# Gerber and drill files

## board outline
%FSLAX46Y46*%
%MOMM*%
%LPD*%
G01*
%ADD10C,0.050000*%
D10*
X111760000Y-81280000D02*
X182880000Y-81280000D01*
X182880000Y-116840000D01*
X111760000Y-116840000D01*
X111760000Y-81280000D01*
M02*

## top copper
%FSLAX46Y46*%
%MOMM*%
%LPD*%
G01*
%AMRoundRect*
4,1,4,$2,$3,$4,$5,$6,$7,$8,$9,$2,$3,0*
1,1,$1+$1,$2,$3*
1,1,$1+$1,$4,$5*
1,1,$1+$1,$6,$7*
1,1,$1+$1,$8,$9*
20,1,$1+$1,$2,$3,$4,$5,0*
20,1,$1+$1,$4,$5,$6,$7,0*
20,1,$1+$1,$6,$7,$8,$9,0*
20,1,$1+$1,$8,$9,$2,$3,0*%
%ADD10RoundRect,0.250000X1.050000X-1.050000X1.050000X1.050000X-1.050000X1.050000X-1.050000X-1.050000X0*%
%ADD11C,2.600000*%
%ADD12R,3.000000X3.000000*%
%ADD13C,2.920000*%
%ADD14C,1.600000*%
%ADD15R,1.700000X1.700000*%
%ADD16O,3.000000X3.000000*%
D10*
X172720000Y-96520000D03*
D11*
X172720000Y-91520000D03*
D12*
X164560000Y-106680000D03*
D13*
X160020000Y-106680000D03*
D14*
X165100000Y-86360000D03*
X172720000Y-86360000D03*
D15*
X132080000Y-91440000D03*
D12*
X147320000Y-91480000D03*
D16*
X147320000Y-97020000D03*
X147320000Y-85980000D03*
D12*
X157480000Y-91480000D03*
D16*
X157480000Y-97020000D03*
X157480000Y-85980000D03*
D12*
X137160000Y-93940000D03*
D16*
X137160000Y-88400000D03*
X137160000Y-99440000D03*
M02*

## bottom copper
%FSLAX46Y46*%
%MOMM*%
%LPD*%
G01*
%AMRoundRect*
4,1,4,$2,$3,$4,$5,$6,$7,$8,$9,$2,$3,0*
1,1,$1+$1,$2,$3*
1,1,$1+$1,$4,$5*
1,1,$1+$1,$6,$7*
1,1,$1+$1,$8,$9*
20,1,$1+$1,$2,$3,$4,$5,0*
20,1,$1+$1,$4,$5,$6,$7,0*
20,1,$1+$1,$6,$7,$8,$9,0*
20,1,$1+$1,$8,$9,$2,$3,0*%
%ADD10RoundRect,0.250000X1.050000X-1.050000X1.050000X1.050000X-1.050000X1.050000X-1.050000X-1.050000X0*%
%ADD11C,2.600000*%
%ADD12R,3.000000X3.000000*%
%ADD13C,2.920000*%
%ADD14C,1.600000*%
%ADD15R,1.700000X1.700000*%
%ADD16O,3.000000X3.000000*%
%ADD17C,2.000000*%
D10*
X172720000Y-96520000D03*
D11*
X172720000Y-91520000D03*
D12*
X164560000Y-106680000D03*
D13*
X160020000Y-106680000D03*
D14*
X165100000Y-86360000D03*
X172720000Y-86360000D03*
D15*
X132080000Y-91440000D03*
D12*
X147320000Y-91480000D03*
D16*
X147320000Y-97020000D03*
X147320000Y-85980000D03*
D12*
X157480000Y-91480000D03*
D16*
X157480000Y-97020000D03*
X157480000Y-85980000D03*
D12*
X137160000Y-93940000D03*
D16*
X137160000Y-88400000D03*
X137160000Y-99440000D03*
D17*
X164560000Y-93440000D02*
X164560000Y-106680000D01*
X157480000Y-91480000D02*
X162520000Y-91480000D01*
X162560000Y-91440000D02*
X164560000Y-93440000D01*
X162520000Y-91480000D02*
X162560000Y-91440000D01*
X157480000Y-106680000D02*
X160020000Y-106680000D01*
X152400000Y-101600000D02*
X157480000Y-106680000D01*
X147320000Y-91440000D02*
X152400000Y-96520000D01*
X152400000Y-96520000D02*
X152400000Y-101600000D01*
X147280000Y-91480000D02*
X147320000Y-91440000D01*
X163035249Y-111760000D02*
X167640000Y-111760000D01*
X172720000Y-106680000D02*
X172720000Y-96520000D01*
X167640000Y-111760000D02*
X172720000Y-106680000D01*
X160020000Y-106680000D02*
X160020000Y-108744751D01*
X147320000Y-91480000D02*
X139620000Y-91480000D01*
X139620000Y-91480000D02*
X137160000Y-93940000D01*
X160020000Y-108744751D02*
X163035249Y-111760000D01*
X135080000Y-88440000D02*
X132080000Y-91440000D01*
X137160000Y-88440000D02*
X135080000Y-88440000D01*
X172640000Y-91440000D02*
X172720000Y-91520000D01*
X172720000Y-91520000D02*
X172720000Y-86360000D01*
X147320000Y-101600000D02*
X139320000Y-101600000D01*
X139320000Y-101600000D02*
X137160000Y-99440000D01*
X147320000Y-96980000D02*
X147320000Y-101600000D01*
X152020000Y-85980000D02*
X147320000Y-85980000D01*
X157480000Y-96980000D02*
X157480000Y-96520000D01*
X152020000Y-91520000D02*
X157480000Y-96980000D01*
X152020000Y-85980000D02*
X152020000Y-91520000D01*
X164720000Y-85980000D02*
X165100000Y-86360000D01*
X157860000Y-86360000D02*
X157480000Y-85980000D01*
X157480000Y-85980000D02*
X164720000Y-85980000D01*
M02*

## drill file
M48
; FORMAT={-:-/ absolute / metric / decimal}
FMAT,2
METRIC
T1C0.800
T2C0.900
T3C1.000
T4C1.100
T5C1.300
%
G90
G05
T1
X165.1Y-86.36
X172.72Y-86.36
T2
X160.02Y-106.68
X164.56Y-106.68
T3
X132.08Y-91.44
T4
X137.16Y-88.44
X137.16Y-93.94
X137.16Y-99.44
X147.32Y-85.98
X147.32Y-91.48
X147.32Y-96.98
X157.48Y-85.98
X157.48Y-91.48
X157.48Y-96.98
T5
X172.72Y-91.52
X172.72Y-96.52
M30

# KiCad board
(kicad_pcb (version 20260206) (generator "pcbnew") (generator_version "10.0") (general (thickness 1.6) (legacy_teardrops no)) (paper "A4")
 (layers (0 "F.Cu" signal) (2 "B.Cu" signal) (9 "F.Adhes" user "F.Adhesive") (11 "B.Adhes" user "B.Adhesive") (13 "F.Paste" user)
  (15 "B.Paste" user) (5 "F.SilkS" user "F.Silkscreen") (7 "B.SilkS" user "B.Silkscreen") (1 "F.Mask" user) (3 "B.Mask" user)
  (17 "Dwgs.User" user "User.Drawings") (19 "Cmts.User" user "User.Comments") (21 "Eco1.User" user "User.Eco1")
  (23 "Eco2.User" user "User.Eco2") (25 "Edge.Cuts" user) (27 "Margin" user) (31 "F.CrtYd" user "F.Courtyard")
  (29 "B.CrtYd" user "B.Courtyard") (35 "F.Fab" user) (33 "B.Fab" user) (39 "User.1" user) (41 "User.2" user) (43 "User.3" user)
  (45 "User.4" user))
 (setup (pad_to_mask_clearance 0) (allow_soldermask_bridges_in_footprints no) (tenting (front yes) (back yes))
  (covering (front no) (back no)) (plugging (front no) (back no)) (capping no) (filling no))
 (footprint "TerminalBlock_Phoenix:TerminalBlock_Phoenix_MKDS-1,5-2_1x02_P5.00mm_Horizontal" (layer "F.Cu") (at 172.72 96.52 90)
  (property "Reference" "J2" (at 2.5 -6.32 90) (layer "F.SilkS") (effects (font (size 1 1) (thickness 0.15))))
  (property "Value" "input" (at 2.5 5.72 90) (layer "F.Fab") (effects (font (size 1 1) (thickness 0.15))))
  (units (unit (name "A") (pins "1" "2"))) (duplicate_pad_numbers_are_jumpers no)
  (pad "1" thru_hole roundrect (at 0 0 90) (size 2.6 2.6) (drill 1.3) (layers "*.Cu" "*.Mask") (remove_unused_layers no)
   (roundrect_rratio 0.096154) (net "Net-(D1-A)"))
  (pad "2" thru_hole circle (at 5 0 90) (size 2.6 2.6) (drill 1.3) (layers "*.Cu" "*.Mask") (remove_unused_layers no) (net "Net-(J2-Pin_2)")))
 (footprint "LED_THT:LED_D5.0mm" (layer "F.Cu") (at 162.56 106.68 180)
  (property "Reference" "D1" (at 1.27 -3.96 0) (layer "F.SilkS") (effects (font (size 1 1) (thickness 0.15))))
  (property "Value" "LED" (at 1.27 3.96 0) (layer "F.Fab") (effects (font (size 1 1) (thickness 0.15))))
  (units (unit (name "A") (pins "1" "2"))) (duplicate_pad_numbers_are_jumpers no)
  (pad "1" thru_hole rect (at -2 0 180) (size 3 3) (drill 0.9) (layers "*.Cu" "*.Mask") (remove_unused_layers no) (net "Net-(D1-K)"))
  (pad "2" thru_hole circle (at 2.54 0 180) (size 2.92 2.92) (drill 0.9) (layers "*.Cu" "*.Mask") (remove_unused_layers no)
   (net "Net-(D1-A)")))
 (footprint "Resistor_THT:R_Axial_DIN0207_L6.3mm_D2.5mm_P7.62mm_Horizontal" (layer "F.Cu") (at 165.1 86.36)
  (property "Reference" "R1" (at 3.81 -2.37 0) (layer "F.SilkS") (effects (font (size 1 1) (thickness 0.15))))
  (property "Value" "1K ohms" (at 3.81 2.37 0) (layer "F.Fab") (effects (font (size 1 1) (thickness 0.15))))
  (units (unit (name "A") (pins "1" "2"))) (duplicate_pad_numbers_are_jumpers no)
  (pad "1" thru_hole circle (at 0 0) (size 1.6 1.6) (drill 0.8) (layers "*.Cu" "*.Mask") (remove_unused_layers no) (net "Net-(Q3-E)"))
  (pad "2" thru_hole circle (at 7.62 0) (size 1.6 1.6) (drill 0.8) (layers "*.Cu" "*.Mask") (remove_unused_layers no) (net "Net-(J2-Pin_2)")))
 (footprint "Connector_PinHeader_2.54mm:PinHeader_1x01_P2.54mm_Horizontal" (layer "F.Cu") (at 132.08 91.44 180)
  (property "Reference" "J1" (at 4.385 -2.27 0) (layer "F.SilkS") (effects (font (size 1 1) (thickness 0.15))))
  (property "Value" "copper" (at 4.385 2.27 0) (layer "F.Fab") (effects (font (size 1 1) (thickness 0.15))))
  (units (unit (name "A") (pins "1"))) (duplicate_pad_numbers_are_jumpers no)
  (pad "1" thru_hole rect (at 0 0 180) (size 1.7 1.7) (drill 1) (layers "*.Cu" "*.Mask") (remove_unused_layers no) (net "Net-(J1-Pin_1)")))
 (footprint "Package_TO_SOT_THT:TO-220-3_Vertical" (layer "F.Cu") (at 147.32 93.98 90)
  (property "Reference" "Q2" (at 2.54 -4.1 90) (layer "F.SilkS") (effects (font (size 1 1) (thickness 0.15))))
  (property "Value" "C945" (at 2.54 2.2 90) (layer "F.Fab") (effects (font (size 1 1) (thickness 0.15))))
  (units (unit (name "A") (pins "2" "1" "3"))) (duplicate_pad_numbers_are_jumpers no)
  (pad "1" thru_hole rect (at 2.5 0 90) (size 3 3) (drill 1.1) (layers "*.Cu" "*.Mask") (remove_unused_layers no) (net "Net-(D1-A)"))
  (pad "2" thru_hole oval (at -3 0 90) (size 3 3) (drill 1.1 (offset -0.04 0)) (layers "*.Cu" "*.Mask") (remove_unused_layers no)
   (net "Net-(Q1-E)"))
  (pad "3" thru_hole oval (at 8 0 90) (size 3 3) (drill 1.1) (layers "*.Cu" "*.Mask") (remove_unused_layers no) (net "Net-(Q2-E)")))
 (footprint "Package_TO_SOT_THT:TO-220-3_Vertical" (layer "F.Cu") (at 157.48 93.98 90)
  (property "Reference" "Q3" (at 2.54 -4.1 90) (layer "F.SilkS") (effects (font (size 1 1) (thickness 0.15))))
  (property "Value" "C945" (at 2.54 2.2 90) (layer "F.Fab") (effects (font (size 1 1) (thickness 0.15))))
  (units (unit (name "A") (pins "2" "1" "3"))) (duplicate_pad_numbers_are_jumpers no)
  (pad "1" thru_hole rect (at 2.5 0 90) (size 3 3) (drill 1.1) (layers "*.Cu" "*.Mask") (remove_unused_layers no) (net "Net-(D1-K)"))
  (pad "2" thru_hole oval (at -3 0 90) (size 3 3) (drill 1.1 (offset -0.04 0)) (layers "*.Cu" "*.Mask") (remove_unused_layers no)
   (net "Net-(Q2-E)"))
  (pad "3" thru_hole oval (at 8 0 90) (size 3 3) (drill 1.1) (layers "*.Cu" "*.Mask") (remove_unused_layers no) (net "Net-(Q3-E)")))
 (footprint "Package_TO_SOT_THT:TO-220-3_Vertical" (layer "F.Cu") (at 137.16 91.44 -90)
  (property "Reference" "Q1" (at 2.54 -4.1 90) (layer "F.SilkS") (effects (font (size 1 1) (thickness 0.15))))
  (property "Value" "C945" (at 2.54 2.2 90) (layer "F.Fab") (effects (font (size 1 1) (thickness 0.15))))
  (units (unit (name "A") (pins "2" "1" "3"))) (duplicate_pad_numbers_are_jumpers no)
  (pad "1" thru_hole rect (at 2.5 0 270) (size 3 3) (drill 1.1) (layers "*.Cu" "*.Mask") (remove_unused_layers no) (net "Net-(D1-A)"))
  (pad "2" thru_hole oval (at -3 0 270) (size 3 3) (drill 1.1 (offset -0.04 0)) (layers "*.Cu" "*.Mask") (remove_unused_layers no)
   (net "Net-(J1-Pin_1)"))
  (pad "3" thru_hole oval (at 8 0 270) (size 3 3) (drill 1.1) (layers "*.Cu" "*.Mask") (remove_unused_layers no) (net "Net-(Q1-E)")))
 (gr_rect (start 111.76 81.28) (end 182.88 116.84) (stroke (width 0.05) (type default)) (fill no) (layer "Edge.Cuts"))
 (segment (start 164.56 93.44) (end 164.56 106.68) (width 2) (layer "B.Cu") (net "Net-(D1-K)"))
 (segment (start 157.48 91.48) (end 162.52 91.48) (width 2) (layer "B.Cu") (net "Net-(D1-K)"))
 (segment (start 162.56 91.44) (end 164.56 93.44) (width 2) (layer "B.Cu") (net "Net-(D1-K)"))
 (segment (start 162.52 91.48) (end 162.56 91.44) (width 2) (layer "B.Cu") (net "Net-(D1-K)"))
 (segment (start 157.48 106.68) (end 160.02 106.68) (width 2) (layer "B.Cu") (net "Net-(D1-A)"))
 (segment (start 152.4 101.6) (end 157.48 106.68) (width 2) (layer "B.Cu") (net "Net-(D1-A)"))
 (segment (start 147.32 91.44) (end 152.4 96.52) (width 2) (layer "B.Cu") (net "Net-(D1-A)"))
 (segment (start 152.4 96.52) (end 152.4 101.6) (width 2) (layer "B.Cu") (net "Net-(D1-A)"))
 (segment (start 147.28 91.48) (end 147.32 91.44) (width 2) (layer "B.Cu") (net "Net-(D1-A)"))
 (segment (start 163.035249 111.76) (end 167.64 111.76) (width 2) (layer "B.Cu") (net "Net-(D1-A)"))
 (segment (start 172.72 106.68) (end 172.72 96.52) (width 2) (layer "B.Cu") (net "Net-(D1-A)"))
 (segment (start 167.64 111.76) (end 172.72 106.68) (width 2) (layer "B.Cu") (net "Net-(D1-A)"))
 (segment (start 160.02 106.68) (end 160.02 108.744751) (width 2) (layer "B.Cu") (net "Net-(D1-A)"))
 (segment (start 147.32 91.48) (end 139.62 91.48) (width 2) (layer "B.Cu") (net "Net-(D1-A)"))
 (segment (start 139.62 91.48) (end 137.16 93.94) (width 2) (layer "B.Cu") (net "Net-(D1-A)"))
 (segment (start 160.02 108.744751) (end 163.035249 111.76) (width 2) (layer "B.Cu") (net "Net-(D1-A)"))
 (segment (start 135.08 88.44) (end 132.08 91.44) (width 2) (layer "B.Cu") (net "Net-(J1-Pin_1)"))
 (segment (start 137.16 88.44) (end 135.08 88.44) (width 2) (layer "B.Cu") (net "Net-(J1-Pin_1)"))
 (segment (start 172.64 91.44) (end 172.72 91.52) (width 2) (layer "B.Cu") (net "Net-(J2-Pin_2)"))
 (segment (start 172.72 91.52) (end 172.72 86.36) (width 2) (layer "B.Cu") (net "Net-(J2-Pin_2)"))
 (segment (start 147.32 101.6) (end 139.32 101.6) (width 2) (layer "B.Cu") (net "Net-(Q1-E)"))
 (segment (start 139.32 101.6) (end 137.16 99.44) (width 2) (layer "B.Cu") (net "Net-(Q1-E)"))
 (segment (start 147.32 96.98) (end 147.32 101.6) (width 2) (layer "B.Cu") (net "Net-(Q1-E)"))
 (segment (start 152.02 85.98) (end 147.32 85.98) (width 2) (layer "B.Cu") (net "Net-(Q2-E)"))
 (segment (start 157.48 96.98) (end 157.48 96.52) (width 2) (layer "B.Cu") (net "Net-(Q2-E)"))
 (segment (start 152.02 91.52) (end 157.48 96.98) (width 2) (layer "B.Cu") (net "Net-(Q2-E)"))
 (segment (start 152.02 85.98) (end 152.02 91.52) (width 2) (layer "B.Cu") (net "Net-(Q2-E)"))
 (segment (start 164.72 85.98) (end 165.1 86.36) (width 2) (layer "B.Cu") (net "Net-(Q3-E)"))
 (segment (start 157.86 86.36) (end 157.48 85.98) (width 2) (layer "B.Cu") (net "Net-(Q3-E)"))
 (segment (start 157.48 85.98) (end 164.72 85.98) (width 2) (layer "B.Cu") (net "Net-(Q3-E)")))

